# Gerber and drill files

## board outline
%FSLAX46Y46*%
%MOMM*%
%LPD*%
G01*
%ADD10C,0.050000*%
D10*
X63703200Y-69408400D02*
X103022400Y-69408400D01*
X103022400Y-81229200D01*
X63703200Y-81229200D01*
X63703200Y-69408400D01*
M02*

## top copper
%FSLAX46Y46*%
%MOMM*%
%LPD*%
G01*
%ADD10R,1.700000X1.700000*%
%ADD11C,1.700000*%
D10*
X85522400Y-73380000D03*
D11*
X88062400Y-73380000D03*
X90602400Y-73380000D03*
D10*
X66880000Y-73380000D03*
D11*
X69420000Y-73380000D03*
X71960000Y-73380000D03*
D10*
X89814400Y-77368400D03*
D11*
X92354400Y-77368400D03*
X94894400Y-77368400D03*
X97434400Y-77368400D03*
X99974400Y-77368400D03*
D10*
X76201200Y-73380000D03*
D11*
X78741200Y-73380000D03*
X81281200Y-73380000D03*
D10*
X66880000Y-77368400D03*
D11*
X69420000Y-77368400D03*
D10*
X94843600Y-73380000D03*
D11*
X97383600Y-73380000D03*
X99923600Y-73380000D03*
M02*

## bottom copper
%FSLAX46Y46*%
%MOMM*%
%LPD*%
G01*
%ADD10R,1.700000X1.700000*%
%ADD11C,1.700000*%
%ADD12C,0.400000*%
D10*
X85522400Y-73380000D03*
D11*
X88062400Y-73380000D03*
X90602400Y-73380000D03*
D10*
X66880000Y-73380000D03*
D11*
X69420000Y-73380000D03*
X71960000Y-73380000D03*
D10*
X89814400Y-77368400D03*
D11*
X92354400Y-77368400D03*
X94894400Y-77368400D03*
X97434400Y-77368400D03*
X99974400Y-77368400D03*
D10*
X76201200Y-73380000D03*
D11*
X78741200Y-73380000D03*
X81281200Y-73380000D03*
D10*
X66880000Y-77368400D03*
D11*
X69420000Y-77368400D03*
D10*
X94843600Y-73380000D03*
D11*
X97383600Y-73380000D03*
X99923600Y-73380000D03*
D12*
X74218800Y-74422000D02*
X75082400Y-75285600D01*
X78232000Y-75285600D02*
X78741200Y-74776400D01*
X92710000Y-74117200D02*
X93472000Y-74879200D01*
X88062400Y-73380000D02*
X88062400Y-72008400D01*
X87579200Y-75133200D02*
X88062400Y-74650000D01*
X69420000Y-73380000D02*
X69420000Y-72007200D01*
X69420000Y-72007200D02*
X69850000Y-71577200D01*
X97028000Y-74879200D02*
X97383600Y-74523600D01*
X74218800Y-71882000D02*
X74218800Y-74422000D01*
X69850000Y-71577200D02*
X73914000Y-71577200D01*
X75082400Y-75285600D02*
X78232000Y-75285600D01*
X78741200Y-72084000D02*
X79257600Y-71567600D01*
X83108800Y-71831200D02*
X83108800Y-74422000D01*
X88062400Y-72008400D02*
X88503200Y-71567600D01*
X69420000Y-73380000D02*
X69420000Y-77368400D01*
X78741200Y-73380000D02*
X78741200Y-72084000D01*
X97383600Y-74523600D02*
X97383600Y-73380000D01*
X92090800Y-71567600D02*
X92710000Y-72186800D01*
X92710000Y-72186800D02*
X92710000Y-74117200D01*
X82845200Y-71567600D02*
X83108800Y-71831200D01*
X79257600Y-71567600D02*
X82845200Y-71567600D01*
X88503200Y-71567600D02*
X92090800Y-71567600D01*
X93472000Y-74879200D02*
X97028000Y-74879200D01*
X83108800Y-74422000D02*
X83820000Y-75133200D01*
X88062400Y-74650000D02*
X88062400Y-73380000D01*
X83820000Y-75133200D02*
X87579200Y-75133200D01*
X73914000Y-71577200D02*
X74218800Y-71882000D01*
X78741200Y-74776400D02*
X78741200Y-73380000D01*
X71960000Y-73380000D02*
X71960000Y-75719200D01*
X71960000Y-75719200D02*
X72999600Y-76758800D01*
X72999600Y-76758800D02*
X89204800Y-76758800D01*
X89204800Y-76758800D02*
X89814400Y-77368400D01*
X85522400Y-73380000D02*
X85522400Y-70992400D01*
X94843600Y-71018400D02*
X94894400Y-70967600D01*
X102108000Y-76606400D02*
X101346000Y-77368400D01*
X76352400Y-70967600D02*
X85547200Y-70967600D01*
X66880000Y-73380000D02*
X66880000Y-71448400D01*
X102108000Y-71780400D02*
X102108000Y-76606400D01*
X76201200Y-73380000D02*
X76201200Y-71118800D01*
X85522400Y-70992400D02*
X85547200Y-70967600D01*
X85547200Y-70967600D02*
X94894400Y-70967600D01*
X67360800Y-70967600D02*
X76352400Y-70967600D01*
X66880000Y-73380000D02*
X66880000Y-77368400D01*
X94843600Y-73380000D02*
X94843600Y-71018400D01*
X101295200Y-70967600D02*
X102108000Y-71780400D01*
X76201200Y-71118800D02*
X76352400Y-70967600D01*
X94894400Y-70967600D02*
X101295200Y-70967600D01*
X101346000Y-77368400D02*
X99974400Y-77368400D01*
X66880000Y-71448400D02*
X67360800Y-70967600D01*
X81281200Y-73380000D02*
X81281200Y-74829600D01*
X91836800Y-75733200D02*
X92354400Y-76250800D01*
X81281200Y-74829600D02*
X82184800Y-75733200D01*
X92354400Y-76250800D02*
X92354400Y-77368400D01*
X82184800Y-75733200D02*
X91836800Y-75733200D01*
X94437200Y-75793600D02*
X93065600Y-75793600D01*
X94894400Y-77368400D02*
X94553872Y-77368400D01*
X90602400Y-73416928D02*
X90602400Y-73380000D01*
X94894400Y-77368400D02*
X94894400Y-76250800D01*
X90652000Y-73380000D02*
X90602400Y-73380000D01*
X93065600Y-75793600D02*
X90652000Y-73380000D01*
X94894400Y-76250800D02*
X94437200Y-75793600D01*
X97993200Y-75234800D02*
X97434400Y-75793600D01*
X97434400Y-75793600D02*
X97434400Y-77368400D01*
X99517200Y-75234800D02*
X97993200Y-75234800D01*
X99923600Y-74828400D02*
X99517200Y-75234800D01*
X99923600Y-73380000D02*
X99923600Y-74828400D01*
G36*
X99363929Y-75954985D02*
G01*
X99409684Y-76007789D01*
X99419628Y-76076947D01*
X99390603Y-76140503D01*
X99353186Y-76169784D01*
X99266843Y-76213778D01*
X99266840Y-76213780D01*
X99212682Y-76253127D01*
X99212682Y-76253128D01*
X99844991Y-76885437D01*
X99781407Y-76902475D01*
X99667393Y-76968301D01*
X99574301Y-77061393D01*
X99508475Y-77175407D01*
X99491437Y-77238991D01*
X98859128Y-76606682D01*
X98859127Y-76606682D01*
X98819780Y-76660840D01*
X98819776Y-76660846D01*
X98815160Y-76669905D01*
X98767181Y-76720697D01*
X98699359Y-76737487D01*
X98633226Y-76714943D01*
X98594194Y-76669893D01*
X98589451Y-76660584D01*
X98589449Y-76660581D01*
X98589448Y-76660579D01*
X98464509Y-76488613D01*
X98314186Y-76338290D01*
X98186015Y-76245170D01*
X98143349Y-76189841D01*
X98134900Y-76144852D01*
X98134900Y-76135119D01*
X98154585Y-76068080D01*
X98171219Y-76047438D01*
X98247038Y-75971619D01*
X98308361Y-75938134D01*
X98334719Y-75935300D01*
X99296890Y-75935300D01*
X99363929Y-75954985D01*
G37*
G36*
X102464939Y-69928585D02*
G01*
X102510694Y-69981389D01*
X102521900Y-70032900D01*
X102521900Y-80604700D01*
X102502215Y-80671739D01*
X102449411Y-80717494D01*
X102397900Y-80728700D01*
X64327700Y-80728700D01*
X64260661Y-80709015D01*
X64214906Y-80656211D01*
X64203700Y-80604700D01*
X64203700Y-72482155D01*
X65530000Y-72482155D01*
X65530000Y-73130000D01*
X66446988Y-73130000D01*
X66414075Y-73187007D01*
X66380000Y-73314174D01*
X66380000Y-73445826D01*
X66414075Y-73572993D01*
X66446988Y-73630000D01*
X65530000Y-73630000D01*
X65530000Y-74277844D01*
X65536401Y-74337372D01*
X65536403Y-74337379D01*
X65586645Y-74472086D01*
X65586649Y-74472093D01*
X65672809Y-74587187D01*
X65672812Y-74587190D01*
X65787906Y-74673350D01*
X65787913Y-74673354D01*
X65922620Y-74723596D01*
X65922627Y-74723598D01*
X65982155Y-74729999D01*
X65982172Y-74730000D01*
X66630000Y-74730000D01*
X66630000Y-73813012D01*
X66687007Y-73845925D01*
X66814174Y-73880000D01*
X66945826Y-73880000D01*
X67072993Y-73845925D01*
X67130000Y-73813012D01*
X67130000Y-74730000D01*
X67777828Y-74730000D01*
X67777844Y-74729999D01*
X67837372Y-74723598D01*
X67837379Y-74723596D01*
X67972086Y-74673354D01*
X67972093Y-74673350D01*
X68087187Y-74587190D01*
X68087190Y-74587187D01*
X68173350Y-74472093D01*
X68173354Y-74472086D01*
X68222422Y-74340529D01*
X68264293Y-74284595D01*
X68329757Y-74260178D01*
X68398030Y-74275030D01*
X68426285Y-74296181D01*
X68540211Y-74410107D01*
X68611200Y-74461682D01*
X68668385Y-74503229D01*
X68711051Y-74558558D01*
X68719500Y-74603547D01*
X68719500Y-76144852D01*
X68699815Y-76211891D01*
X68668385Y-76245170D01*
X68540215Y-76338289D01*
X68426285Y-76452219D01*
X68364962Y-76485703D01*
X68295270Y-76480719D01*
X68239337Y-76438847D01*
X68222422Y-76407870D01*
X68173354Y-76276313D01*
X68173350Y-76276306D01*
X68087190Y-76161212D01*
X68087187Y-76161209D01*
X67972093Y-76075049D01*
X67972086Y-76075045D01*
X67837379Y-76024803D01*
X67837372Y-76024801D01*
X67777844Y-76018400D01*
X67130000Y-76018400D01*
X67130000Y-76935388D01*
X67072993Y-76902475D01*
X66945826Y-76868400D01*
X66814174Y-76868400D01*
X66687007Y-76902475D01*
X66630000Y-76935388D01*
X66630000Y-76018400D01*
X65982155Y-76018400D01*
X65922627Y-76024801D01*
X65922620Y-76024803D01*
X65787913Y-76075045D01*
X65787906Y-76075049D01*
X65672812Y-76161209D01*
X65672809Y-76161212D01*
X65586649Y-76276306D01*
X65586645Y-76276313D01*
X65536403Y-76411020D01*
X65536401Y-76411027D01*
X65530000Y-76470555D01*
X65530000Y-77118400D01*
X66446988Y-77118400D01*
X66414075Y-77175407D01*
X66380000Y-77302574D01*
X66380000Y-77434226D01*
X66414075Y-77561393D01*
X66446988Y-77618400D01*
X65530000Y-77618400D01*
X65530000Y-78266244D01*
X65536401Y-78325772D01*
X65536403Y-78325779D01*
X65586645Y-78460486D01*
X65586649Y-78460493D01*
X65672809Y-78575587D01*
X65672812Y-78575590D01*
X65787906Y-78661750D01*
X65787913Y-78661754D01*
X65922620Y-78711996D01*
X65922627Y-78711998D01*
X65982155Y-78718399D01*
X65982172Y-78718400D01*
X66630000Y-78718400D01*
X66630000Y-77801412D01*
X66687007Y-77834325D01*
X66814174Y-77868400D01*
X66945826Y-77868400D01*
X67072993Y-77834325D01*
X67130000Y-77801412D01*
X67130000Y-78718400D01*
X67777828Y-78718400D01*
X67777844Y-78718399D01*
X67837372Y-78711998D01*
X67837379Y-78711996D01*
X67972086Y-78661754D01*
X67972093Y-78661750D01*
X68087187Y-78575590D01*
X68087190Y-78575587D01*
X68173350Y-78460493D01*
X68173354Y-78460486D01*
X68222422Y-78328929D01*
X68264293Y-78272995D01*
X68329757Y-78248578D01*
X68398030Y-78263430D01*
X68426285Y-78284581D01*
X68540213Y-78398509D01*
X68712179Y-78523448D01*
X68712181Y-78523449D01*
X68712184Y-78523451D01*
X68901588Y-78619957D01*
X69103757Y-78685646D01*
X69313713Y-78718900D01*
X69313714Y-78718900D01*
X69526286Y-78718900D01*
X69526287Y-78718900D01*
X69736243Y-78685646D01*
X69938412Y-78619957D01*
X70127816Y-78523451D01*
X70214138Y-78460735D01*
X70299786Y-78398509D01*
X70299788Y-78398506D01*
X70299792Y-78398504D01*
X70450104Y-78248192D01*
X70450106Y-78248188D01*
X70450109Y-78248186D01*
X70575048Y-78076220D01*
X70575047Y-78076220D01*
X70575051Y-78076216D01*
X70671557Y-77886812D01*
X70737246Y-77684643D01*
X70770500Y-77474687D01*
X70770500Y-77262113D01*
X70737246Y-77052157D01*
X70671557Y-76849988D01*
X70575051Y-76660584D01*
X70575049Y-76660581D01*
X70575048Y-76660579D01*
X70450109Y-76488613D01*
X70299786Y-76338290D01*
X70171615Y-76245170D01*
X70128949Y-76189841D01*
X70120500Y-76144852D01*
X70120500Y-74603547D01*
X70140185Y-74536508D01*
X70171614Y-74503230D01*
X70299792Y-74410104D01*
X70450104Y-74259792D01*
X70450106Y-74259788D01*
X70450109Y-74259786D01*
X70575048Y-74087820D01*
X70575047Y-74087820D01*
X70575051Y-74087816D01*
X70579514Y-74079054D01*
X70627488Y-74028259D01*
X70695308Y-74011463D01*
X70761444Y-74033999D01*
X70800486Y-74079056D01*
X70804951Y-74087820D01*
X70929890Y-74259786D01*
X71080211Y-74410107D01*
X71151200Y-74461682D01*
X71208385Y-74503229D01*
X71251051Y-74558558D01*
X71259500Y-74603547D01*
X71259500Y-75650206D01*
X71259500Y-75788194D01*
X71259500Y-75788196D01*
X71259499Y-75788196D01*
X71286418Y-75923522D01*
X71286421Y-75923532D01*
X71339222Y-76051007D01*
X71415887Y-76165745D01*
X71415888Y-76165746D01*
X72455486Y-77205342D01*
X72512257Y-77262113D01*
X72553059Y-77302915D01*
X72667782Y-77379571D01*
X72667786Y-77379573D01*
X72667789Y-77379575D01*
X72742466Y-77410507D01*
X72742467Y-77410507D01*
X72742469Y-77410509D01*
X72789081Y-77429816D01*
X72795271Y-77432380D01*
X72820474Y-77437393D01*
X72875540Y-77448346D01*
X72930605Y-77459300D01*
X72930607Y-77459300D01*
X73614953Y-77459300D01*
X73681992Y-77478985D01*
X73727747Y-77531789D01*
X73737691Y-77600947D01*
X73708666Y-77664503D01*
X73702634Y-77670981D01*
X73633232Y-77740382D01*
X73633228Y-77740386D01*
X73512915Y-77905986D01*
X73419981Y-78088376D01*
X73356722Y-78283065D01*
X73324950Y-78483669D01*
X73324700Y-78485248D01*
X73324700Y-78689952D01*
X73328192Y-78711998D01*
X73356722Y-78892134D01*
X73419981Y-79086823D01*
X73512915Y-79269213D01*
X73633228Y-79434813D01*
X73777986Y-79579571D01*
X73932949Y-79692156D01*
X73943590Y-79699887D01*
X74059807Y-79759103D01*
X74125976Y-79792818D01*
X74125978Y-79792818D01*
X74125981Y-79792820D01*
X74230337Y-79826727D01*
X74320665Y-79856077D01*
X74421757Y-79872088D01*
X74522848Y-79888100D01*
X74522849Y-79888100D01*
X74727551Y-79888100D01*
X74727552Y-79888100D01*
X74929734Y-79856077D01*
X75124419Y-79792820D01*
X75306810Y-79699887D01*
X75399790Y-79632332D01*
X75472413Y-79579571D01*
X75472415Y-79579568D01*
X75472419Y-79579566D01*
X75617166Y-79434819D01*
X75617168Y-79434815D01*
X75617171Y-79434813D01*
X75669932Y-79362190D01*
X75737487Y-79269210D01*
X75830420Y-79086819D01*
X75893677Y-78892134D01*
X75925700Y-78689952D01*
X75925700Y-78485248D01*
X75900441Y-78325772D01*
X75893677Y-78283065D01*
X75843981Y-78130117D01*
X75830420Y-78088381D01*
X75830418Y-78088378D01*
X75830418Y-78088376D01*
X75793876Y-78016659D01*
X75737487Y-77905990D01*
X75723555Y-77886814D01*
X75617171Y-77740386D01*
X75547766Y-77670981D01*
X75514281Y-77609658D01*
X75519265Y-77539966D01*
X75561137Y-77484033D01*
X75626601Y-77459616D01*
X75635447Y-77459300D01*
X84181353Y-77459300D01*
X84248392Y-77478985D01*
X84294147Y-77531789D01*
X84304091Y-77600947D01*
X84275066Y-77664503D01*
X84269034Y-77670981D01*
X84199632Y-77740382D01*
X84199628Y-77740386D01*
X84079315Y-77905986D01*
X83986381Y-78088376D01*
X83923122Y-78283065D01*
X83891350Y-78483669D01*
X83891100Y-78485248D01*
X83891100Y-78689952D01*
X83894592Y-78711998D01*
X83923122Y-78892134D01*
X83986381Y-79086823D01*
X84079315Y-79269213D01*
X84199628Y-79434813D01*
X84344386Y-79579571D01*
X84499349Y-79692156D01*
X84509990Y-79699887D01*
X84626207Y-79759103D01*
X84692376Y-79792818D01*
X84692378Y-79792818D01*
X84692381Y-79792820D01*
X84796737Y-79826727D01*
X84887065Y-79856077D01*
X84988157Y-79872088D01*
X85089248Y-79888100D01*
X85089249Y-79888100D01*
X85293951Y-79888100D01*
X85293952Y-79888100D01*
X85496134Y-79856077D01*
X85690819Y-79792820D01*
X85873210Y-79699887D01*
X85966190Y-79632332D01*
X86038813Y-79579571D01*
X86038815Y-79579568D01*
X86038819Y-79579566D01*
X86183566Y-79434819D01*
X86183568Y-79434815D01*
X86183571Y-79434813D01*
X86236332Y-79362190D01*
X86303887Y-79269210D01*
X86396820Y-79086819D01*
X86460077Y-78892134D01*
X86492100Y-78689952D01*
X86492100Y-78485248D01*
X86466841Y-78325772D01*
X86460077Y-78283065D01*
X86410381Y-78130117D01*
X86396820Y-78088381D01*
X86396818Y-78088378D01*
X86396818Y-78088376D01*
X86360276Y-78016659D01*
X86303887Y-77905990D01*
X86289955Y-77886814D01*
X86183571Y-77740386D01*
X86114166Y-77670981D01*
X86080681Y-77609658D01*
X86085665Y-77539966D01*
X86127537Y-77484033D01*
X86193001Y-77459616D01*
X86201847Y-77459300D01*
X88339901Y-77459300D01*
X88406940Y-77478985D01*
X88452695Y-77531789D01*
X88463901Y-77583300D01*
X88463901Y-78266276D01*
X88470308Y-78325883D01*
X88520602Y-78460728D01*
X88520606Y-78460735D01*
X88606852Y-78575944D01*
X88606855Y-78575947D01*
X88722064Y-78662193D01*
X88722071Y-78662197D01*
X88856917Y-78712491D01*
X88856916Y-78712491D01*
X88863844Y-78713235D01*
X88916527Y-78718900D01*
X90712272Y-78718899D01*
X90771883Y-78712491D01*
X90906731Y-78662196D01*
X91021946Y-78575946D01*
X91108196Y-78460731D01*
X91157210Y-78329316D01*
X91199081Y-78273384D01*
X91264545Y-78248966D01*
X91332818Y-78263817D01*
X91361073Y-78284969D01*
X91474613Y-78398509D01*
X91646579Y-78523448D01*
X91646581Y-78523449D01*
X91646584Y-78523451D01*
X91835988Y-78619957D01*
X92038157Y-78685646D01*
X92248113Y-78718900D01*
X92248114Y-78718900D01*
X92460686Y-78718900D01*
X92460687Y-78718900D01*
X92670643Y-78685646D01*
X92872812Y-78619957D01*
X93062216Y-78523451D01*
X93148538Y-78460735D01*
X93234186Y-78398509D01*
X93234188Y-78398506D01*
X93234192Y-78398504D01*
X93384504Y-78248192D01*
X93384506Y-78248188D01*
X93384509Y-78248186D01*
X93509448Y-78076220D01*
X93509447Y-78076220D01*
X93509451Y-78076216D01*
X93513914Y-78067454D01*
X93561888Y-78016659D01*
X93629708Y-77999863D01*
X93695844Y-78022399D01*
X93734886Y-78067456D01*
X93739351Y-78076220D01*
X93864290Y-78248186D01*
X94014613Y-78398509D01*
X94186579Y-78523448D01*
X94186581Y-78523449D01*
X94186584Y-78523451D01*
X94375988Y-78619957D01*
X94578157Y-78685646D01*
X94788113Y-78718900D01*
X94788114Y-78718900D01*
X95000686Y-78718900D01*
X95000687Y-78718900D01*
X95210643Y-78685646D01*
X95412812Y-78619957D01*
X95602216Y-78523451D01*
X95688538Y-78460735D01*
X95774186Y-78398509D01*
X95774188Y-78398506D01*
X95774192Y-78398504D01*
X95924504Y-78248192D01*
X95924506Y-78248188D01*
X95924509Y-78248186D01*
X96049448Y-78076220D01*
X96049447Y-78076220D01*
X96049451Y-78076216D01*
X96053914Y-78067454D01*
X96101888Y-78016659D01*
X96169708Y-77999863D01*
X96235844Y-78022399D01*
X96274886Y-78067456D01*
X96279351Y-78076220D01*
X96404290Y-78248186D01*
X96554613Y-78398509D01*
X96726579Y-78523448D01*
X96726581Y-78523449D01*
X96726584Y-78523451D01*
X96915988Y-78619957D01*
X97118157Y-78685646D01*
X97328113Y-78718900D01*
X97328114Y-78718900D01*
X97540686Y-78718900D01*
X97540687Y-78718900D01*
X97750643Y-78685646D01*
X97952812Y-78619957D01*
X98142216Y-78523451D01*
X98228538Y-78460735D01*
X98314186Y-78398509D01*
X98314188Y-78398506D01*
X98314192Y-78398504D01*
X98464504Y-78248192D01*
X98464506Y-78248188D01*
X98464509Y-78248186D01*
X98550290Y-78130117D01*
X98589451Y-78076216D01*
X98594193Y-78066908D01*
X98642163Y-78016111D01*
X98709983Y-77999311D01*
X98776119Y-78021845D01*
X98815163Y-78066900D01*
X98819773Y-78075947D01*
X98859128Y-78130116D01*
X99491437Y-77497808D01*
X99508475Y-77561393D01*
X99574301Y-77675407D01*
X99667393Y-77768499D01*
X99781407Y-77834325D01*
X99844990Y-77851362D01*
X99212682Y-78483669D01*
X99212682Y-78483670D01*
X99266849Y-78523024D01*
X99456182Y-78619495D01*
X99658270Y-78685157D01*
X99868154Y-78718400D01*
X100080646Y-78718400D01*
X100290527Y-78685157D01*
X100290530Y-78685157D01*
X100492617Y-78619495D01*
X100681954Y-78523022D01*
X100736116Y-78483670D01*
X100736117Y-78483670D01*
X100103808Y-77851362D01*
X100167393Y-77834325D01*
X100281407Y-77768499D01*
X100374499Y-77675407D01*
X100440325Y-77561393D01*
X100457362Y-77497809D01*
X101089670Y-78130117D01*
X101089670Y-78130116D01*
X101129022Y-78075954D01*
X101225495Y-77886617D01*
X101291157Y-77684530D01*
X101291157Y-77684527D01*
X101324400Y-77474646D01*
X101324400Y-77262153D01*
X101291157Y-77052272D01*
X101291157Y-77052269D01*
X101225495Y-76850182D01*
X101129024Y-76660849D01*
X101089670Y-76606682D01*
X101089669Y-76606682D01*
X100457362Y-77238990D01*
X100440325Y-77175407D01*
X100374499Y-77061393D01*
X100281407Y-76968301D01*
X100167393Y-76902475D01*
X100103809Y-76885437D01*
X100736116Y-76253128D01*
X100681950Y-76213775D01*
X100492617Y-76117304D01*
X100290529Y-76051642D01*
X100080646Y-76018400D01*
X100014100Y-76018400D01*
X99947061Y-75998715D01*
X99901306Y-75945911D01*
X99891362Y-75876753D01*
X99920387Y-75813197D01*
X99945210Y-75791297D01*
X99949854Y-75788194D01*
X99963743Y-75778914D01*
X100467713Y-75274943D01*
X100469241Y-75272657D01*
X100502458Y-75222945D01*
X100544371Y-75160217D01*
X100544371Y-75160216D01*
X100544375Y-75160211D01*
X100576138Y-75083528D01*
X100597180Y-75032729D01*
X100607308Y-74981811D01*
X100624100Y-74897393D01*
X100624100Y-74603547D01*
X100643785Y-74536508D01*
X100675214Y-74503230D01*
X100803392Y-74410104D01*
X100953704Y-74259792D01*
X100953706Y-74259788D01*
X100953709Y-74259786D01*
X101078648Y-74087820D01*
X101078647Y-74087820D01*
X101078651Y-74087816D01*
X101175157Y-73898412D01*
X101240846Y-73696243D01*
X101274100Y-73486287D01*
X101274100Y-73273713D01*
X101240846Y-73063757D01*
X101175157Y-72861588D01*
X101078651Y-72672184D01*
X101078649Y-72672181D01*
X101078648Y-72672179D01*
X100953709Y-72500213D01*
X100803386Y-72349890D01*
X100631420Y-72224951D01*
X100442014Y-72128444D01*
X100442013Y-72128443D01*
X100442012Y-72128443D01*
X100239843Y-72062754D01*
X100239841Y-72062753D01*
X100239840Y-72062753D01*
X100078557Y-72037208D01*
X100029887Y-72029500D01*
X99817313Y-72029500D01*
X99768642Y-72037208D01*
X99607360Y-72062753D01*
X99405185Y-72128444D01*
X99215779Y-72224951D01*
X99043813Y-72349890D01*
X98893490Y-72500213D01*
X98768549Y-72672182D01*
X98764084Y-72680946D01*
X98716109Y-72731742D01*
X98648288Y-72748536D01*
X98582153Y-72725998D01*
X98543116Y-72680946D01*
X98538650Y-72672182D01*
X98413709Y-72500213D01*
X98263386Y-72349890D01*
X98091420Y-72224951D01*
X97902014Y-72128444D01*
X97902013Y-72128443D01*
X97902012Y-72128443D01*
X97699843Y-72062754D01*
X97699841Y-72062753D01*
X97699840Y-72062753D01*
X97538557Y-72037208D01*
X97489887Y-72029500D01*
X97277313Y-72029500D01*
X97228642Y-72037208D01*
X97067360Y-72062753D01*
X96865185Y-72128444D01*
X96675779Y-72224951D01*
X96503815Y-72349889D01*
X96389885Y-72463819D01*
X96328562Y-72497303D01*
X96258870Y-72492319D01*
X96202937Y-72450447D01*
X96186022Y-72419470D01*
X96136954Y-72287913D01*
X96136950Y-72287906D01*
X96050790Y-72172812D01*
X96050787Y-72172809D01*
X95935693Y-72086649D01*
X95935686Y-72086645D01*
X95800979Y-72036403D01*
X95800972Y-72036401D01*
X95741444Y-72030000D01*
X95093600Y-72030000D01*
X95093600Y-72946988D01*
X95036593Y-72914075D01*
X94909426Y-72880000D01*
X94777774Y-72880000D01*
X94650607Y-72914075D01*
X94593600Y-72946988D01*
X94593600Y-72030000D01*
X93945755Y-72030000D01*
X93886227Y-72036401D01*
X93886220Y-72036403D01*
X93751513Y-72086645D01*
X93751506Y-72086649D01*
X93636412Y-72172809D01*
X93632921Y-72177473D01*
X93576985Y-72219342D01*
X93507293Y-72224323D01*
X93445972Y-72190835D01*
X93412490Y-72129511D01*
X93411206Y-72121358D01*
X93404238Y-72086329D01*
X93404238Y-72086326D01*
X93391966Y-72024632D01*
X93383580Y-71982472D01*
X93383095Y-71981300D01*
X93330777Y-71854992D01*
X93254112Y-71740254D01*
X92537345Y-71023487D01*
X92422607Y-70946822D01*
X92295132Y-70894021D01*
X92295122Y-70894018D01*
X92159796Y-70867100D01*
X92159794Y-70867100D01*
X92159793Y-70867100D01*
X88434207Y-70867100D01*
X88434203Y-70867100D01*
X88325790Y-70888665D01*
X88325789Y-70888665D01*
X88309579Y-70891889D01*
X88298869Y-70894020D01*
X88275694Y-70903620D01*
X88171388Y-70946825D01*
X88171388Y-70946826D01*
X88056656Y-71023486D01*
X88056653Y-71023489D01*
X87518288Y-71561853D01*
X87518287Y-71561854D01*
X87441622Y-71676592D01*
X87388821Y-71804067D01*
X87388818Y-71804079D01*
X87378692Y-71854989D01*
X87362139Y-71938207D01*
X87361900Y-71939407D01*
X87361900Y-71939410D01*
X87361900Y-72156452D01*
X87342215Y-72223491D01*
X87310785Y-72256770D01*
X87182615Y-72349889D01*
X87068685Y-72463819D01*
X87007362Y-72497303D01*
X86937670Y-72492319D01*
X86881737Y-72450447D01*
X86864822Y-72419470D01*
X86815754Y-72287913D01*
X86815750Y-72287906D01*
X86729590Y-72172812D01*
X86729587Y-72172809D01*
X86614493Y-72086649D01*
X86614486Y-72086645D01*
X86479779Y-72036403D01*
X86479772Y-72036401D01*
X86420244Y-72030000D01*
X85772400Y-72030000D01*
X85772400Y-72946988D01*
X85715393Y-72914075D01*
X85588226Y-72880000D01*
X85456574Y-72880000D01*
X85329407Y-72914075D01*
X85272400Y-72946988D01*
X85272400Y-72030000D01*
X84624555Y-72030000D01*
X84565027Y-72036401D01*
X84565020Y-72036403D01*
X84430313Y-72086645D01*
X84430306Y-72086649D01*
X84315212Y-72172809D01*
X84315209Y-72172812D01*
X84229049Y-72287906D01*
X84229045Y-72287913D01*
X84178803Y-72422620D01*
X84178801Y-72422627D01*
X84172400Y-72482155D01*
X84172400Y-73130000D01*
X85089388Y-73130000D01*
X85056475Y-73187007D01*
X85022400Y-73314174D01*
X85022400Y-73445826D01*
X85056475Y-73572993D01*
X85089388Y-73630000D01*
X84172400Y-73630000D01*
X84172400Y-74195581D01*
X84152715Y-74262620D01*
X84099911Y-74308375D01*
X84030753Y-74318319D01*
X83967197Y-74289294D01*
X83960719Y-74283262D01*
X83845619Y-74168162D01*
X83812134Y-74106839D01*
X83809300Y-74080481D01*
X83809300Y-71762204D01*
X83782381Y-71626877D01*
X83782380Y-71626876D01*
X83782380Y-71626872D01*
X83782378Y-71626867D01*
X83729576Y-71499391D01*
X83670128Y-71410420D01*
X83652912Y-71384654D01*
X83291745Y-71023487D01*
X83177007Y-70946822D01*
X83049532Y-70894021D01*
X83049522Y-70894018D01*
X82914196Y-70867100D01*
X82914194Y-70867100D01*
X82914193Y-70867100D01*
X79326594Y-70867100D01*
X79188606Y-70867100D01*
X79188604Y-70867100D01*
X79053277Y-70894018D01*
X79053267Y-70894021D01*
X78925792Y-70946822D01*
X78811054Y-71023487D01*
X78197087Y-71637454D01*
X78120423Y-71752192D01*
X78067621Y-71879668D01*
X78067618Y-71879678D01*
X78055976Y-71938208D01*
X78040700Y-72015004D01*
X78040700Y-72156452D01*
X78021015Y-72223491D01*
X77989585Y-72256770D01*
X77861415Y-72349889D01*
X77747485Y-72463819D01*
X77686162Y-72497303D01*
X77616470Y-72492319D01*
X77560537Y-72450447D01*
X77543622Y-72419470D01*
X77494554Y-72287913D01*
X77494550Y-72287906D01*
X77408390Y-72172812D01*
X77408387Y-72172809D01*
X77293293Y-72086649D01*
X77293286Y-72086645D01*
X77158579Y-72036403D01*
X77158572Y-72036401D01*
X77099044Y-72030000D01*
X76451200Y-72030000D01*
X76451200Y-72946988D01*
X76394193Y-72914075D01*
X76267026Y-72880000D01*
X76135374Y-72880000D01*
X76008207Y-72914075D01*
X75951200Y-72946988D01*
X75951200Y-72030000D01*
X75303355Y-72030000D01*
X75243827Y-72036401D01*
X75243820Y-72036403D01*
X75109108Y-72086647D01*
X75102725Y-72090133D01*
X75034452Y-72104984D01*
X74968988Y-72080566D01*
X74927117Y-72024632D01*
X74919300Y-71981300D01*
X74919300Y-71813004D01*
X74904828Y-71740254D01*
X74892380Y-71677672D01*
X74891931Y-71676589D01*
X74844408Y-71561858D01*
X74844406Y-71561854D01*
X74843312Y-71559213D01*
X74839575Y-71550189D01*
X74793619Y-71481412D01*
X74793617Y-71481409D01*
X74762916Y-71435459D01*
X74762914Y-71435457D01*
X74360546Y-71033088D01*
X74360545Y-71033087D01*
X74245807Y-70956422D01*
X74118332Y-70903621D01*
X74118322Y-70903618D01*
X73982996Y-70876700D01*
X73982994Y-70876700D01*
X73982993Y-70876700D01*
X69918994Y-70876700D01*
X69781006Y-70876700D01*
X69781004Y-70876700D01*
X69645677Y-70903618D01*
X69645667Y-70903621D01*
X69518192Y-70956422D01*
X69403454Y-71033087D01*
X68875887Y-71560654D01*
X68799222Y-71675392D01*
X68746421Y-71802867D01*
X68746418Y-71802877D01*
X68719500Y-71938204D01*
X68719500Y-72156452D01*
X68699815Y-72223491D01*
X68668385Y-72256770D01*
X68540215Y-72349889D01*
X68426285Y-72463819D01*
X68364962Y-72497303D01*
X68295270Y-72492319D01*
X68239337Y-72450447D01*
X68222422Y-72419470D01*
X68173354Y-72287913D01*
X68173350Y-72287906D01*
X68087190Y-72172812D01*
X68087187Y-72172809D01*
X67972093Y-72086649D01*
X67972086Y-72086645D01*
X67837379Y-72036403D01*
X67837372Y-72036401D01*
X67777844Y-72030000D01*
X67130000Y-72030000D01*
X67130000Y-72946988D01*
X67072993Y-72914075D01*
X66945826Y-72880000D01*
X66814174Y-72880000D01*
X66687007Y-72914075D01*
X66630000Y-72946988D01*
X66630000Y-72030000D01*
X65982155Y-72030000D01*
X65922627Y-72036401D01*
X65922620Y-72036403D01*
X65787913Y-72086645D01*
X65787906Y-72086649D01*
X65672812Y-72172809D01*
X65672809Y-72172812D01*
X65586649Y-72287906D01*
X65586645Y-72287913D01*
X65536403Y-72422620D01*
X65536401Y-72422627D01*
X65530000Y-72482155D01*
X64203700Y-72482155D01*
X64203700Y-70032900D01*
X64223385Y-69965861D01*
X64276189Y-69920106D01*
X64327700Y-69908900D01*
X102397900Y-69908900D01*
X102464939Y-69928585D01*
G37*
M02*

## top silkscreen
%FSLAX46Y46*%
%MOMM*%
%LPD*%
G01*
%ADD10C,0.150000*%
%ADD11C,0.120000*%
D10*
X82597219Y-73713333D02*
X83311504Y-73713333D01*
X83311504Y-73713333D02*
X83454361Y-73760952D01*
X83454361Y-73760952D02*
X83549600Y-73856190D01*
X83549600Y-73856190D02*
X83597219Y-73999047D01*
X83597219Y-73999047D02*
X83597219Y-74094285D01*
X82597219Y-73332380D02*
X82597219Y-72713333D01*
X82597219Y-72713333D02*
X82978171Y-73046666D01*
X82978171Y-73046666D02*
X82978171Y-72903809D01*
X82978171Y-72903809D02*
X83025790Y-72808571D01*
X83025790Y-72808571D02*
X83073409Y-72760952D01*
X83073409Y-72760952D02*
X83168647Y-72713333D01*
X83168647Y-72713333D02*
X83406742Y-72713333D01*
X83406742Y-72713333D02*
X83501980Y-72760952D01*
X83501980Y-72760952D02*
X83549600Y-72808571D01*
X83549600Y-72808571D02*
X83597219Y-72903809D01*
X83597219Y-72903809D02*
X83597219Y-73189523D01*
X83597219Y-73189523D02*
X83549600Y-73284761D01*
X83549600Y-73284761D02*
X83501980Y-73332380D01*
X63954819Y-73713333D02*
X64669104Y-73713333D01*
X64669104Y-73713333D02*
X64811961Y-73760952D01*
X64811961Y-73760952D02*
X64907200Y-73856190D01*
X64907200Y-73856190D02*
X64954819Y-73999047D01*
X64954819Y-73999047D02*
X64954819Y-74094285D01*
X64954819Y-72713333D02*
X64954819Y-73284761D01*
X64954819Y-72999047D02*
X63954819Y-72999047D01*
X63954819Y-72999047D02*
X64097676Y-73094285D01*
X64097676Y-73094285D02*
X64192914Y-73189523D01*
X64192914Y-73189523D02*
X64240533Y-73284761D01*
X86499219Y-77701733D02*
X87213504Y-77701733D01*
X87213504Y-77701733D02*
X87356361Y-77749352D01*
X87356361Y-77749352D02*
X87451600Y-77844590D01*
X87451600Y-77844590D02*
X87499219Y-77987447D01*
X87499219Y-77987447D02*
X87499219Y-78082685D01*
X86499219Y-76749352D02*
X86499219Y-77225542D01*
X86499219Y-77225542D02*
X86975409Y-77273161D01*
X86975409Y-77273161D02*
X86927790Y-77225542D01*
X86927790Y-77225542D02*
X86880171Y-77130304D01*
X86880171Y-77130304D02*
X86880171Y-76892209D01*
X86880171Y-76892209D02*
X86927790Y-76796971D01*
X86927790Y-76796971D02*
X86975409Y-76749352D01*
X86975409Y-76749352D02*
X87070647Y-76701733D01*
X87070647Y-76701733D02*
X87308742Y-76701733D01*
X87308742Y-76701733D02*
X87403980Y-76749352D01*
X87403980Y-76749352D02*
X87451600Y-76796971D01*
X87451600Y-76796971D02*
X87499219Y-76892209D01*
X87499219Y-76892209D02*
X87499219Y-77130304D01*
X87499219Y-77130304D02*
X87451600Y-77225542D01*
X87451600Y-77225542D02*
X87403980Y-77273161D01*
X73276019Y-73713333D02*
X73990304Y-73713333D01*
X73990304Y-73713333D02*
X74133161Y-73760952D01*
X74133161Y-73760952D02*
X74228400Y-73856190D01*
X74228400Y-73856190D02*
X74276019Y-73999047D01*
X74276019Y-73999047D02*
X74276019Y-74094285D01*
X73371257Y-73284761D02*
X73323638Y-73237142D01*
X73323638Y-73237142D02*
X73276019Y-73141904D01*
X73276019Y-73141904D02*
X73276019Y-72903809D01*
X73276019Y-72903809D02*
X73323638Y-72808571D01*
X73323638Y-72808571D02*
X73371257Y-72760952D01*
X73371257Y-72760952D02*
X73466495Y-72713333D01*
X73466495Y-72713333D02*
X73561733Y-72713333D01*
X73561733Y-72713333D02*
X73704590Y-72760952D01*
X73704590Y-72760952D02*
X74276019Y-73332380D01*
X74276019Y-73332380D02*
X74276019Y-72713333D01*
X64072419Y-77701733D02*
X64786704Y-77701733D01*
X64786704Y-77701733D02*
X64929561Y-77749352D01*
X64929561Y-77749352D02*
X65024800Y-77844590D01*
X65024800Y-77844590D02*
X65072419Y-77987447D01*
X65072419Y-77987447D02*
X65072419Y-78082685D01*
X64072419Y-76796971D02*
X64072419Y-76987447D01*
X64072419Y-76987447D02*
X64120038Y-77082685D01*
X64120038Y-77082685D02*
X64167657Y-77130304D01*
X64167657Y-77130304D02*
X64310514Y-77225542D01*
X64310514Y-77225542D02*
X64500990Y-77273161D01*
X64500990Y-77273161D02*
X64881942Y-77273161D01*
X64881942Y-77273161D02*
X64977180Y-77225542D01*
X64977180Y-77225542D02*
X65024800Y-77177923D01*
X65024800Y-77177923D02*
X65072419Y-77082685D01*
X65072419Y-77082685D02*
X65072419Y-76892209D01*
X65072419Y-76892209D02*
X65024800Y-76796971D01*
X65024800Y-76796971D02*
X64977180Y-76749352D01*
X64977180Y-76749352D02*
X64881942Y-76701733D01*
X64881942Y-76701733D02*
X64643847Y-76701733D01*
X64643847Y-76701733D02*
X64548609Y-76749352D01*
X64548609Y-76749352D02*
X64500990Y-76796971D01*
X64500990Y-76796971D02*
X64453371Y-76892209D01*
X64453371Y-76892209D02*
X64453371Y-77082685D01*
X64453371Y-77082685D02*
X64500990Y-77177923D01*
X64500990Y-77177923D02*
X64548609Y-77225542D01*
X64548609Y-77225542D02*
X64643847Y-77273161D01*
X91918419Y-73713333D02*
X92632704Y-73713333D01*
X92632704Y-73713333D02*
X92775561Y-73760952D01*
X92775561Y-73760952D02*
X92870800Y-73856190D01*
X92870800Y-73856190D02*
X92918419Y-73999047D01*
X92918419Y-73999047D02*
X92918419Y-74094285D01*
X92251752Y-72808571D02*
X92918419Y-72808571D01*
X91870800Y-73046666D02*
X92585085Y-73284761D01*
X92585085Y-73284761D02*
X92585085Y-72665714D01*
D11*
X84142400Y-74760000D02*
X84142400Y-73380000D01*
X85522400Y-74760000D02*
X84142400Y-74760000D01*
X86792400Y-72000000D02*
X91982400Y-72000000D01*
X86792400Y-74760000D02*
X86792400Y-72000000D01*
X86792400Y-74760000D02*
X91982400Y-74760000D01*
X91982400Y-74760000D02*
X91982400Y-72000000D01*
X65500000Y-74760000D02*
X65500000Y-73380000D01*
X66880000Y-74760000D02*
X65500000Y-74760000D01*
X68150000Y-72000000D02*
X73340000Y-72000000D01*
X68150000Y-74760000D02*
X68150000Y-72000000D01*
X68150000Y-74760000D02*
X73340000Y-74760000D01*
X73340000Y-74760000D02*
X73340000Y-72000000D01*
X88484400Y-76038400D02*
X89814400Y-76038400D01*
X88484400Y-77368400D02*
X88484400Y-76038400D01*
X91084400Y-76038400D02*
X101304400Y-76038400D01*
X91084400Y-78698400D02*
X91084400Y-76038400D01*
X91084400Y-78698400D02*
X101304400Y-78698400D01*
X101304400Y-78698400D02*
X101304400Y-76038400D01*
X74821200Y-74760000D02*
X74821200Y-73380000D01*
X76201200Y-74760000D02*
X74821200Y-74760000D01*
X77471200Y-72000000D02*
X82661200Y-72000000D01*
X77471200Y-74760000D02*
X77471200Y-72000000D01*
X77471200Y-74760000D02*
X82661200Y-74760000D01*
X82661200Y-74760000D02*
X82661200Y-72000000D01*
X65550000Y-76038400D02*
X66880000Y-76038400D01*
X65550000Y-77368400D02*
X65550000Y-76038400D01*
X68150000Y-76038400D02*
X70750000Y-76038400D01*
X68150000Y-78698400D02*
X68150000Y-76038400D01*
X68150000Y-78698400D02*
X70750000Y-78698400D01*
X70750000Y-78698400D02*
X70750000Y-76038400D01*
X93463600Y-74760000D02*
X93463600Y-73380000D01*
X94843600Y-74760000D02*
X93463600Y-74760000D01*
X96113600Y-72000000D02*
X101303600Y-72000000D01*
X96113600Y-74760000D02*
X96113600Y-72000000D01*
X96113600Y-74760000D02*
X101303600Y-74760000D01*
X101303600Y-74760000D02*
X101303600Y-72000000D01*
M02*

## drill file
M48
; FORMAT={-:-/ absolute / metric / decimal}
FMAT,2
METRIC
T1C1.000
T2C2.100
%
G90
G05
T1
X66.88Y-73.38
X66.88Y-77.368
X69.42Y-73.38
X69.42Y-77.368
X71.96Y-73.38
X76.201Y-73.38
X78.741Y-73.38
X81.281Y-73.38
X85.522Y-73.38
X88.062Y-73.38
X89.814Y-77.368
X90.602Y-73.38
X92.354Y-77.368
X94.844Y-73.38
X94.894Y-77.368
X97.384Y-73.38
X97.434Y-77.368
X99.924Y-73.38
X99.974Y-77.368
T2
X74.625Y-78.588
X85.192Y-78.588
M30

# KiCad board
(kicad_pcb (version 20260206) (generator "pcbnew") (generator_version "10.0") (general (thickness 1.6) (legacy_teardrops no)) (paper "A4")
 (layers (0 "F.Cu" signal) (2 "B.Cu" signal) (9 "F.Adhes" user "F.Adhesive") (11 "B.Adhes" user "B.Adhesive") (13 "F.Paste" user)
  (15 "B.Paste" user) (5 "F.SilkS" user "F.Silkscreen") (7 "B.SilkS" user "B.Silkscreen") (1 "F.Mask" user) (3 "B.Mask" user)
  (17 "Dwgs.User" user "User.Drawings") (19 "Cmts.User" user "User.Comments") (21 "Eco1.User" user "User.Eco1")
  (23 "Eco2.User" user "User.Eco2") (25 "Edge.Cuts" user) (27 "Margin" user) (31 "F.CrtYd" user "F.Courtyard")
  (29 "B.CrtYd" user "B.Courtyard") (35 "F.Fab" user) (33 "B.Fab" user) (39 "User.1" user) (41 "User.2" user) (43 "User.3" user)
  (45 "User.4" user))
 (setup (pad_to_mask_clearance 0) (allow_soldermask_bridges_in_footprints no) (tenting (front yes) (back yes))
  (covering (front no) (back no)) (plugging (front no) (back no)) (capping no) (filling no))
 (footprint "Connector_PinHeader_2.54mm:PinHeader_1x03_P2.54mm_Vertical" (layer "F.Cu") (at 85.5224 73.38 90)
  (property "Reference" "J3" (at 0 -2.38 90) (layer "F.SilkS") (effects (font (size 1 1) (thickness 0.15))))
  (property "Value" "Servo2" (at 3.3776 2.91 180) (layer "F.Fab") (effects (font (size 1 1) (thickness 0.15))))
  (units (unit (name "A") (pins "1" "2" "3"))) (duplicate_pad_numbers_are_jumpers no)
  (fp_line (start -1.38 -1.38) (end 0 -1.38) (stroke (width 0.12) (type solid)) (layer "F.SilkS"))
  (fp_line (start -1.38 0) (end -1.38 -1.38) (stroke (width 0.12) (type solid)) (layer "F.SilkS"))
  (fp_line (start 1.38 1.27) (end 1.38 6.46) (stroke (width 0.12) (type solid)) (layer "F.SilkS"))
  (fp_line (start -1.38 1.27) (end 1.38 1.27) (stroke (width 0.12) (type solid)) (layer "F.SilkS"))
  (fp_line (start -1.38 1.27) (end -1.38 6.46) (stroke (width 0.12) (type solid)) (layer "F.SilkS"))
  (fp_line (start -1.38 6.46) (end 1.38 6.46) (stroke (width 0.12) (type solid)) (layer "F.SilkS"))
  (pad "1" thru_hole rect (at 0 0 90) (size 1.7 1.7) (drill 1) (layers "*.Cu" "*.Mask") (remove_unused_layers no) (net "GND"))
  (pad "2" thru_hole circle (at 0 2.54 90) (size 1.7 1.7) (drill 1) (layers "*.Cu" "*.Mask") (remove_unused_layers no) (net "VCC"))
  (pad "3" thru_hole circle (at 0 5.08 90) (size 1.7 1.7) (drill 1) (layers "*.Cu" "*.Mask") (remove_unused_layers no) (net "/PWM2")))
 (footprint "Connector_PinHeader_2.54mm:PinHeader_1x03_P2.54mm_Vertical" (layer "F.Cu") (at 66.88 73.38 90)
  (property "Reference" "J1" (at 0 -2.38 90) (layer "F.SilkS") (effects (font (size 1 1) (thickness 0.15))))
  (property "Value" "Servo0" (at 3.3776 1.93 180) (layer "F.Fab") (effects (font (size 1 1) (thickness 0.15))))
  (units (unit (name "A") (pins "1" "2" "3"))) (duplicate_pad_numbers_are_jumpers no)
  (fp_line (start -1.38 -1.38) (end 0 -1.38) (stroke (width 0.12) (type solid)) (layer "F.SilkS"))
  (fp_line (start -1.38 0) (end -1.38 -1.38) (stroke (width 0.12) (type solid)) (layer "F.SilkS"))
  (fp_line (start 1.38 1.27) (end 1.38 6.46) (stroke (width 0.12) (type solid)) (layer "F.SilkS"))
  (fp_line (start -1.38 1.27) (end 1.38 1.27) (stroke (width 0.12) (type solid)) (layer "F.SilkS"))
  (fp_line (start -1.38 1.27) (end -1.38 6.46) (stroke (width 0.12) (type solid)) (layer "F.SilkS"))
  (fp_line (start -1.38 6.46) (end 1.38 6.46) (stroke (width 0.12) (type solid)) (layer "F.SilkS"))
  (pad "1" thru_hole rect (at 0 0 90) (size 1.7 1.7) (drill 1) (layers "*.Cu" "*.Mask") (remove_unused_layers no) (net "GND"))
  (pad "2" thru_hole circle (at 0 2.54 90) (size 1.7 1.7) (drill 1) (layers "*.Cu" "*.Mask") (remove_unused_layers no) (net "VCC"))
  (pad "3" thru_hole circle (at 0 5.08 90) (size 1.7 1.7) (drill 1) (layers "*.Cu" "*.Mask") (remove_unused_layers no) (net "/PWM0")))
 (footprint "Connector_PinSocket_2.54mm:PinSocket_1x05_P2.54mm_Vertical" (layer "F.Cu") (at 89.8144 77.3684 90)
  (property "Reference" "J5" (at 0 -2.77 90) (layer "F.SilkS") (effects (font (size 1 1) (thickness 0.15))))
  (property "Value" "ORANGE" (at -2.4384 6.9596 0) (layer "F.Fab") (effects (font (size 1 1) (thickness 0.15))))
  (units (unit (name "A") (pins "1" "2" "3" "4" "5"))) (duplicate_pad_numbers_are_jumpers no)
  (fp_line (start 1.33 -1.33) (end 1.33 0) (stroke (width 0.12) (type solid)) (layer "F.SilkS"))
  (fp_line (start 0 -1.33) (end 1.33 -1.33) (stroke (width 0.12) (type solid)) (layer "F.SilkS"))
  (fp_line (start 1.33 1.27) (end 1.33 11.49) (stroke (width 0.12) (type solid)) (layer "F.SilkS"))
  (fp_line (start -1.33 1.27) (end 1.33 1.27) (stroke (width 0.12) (type solid)) (layer "F.SilkS"))
  (fp_line (start -1.33 1.27) (end -1.33 11.49) (stroke (width 0.12) (type solid)) (layer "F.SilkS"))
  (fp_line (start -1.33 11.49) (end 1.33 11.49) (stroke (width 0.12) (type solid)) (layer "F.SilkS"))
  (pad "1" thru_hole rect (at 0 0 90) (size 1.7 1.7) (drill 1) (layers "*.Cu" "*.Mask") (remove_unused_layers no) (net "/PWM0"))
  (pad "2" thru_hole circle (at 0 2.54 90) (size 1.7 1.7) (drill 1) (layers "*.Cu" "*.Mask") (remove_unused_layers no) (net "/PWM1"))
  (pad "3" thru_hole circle (at 0 5.08 90) (size 1.7 1.7) (drill 1) (layers "*.Cu" "*.Mask") (remove_unused_layers no) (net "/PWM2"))
  (pad "4" thru_hole circle (at 0 7.62 90) (size 1.7 1.7) (drill 1) (layers "*.Cu" "*.Mask") (remove_unused_layers no) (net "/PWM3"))
  (pad "5" thru_hole circle (at 0 10.16 90) (size 1.7 1.7) (drill 1) (layers "*.Cu" "*.Mask") (remove_unused_layers no) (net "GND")))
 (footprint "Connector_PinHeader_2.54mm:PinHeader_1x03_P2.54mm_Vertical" (layer "F.Cu") (at 76.2012 73.38 90)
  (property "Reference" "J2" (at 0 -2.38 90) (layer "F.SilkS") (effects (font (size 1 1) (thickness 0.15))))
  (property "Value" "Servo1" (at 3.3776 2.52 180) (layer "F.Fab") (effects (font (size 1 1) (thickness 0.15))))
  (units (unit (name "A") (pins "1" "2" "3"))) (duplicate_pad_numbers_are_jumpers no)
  (fp_line (start -1.38 -1.38) (end 0 -1.38) (stroke (width 0.12) (type solid)) (layer "F.SilkS"))
  (fp_line (start -1.38 0) (end -1.38 -1.38) (stroke (width 0.12) (type solid)) (layer "F.SilkS"))
  (fp_line (start 1.38 1.27) (end 1.38 6.46) (stroke (width 0.12) (type solid)) (layer "F.SilkS"))
  (fp_line (start -1.38 1.27) (end 1.38 1.27) (stroke (width 0.12) (type solid)) (layer "F.SilkS"))
  (fp_line (start -1.38 1.27) (end -1.38 6.46) (stroke (width 0.12) (type solid)) (layer "F.SilkS"))
  (fp_line (start -1.38 6.46) (end 1.38 6.46) (stroke (width 0.12) (type solid)) (layer "F.SilkS"))
  (pad "1" thru_hole rect (at 0 0 90) (size 1.7 1.7) (drill 1) (layers "*.Cu" "*.Mask") (remove_unused_layers no) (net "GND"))
  (pad "2" thru_hole circle (at 0 2.54 90) (size 1.7 1.7) (drill 1) (layers "*.Cu" "*.Mask") (remove_unused_layers no) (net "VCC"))
  (pad "3" thru_hole circle (at 0 5.08 90) (size 1.7 1.7) (drill 1) (layers "*.Cu" "*.Mask") (remove_unused_layers no) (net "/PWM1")))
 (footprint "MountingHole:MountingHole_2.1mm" (layer "F.Cu") (at 74.6252 78.5876)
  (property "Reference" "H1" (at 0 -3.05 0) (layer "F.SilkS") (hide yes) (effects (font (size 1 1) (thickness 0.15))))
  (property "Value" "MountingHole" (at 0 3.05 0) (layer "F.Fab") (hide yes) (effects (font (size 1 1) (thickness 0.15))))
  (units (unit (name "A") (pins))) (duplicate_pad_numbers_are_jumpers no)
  (pad "" np_thru_hole circle (at 0 0) (size 2.1 2.1) (drill 2.1) (layers "*.Cu" "*.Mask")))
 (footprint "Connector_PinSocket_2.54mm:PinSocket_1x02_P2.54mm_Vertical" (layer "F.Cu") (at 66.88 77.3684 90)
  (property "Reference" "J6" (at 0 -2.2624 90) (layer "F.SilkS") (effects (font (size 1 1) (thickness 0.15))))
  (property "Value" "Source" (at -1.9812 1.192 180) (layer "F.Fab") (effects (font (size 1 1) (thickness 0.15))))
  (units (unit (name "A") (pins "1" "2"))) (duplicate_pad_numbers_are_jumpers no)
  (fp_line (start 1.33 -1.33) (end 1.33 0) (stroke (width 0.12) (type solid)) (layer "F.SilkS"))
  (fp_line (start 0 -1.33) (end 1.33 -1.33) (stroke (width 0.12) (type solid)) (layer "F.SilkS"))
  (fp_line (start 1.33 1.27) (end 1.33 3.87) (stroke (width 0.12) (type solid)) (layer "F.SilkS"))
  (fp_line (start -1.33 1.27) (end 1.33 1.27) (stroke (width 0.12) (type solid)) (layer "F.SilkS"))
  (fp_line (start -1.33 1.27) (end -1.33 3.87) (stroke (width 0.12) (type solid)) (layer "F.SilkS"))
  (fp_line (start -1.33 3.87) (end 1.33 3.87) (stroke (width 0.12) (type solid)) (layer "F.SilkS"))
  (pad "1" thru_hole rect (at 0 0 90) (size 1.7 1.7) (drill 1) (layers "*.Cu" "*.Mask") (remove_unused_layers no) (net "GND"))
  (pad "2" thru_hole circle (at 0 2.54 90) (size 1.7 1.7) (drill 1) (layers "*.Cu" "*.Mask") (remove_unused_layers no) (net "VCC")))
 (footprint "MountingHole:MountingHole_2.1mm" (layer "F.Cu") (at 85.1916 78.5876)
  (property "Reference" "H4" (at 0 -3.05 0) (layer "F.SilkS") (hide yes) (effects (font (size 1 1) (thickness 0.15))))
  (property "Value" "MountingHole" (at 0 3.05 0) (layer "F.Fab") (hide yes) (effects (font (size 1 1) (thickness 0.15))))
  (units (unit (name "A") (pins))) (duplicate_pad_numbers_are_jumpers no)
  (pad "" np_thru_hole circle (at 0 0) (size 2.1 2.1) (drill 2.1) (layers "*.Cu" "*.Mask")))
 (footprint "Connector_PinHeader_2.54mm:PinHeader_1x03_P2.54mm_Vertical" (layer "F.Cu") (at 94.8436 73.38 90)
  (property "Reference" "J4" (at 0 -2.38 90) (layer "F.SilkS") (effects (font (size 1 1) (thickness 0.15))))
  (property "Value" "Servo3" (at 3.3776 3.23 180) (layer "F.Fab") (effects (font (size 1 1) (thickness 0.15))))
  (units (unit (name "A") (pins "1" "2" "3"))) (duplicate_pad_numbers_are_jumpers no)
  (fp_line (start -1.38 -1.38) (end 0 -1.38) (stroke (width 0.12) (type solid)) (layer "F.SilkS"))
  (fp_line (start -1.38 0) (end -1.38 -1.38) (stroke (width 0.12) (type solid)) (layer "F.SilkS"))
  (fp_line (start 1.38 1.27) (end 1.38 6.46) (stroke (width 0.12) (type solid)) (layer "F.SilkS"))
  (fp_line (start -1.38 1.27) (end 1.38 1.27) (stroke (width 0.12) (type solid)) (layer "F.SilkS"))
  (fp_line (start -1.38 1.27) (end -1.38 6.46) (stroke (width 0.12) (type solid)) (layer "F.SilkS"))
  (fp_line (start -1.38 6.46) (end 1.38 6.46) (stroke (width 0.12) (type solid)) (layer "F.SilkS"))
  (pad "1" thru_hole rect (at 0 0 90) (size 1.7 1.7) (drill 1) (layers "*.Cu" "*.Mask") (remove_unused_layers no) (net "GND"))
  (pad "2" thru_hole circle (at 0 2.54 90) (size 1.7 1.7) (drill 1) (layers "*.Cu" "*.Mask") (remove_unused_layers no) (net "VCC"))
  (pad "3" thru_hole circle (at 0 5.08 90) (size 1.7 1.7) (drill 1) (layers "*.Cu" "*.Mask") (remove_unused_layers no) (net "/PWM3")))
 (gr_rect (start 63.7032 69.4084) (end 103.0224 81.2292) (stroke (width 0.05) (type default)) (fill no) (layer "Edge.Cuts"))
 (segment (start 74.2188 74.422) (end 75.0824 75.2856) (width 0.4) (layer "B.Cu") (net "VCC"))
 (segment (start 78.232 75.2856) (end 78.7412 74.7764) (width 0.4) (layer "B.Cu") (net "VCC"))
 (segment (start 92.71 74.1172) (end 93.472 74.8792) (width 0.4) (layer "B.Cu") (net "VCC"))
 (segment (start 88.0624 73.38) (end 88.0624 72.0084) (width 0.4) (layer "B.Cu") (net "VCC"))
 (segment (start 87.5792 75.1332) (end 88.0624 74.65) (width 0.4) (layer "B.Cu") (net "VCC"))
 (segment (start 69.42 73.38) (end 69.42 72.0072) (width 0.4) (layer "B.Cu") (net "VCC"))
 (segment (start 69.42 72.0072) (end 69.85 71.5772) (width 0.4) (layer "B.Cu") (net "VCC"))
 (segment (start 97.028 74.8792) (end 97.3836 74.5236) (width 0.4) (layer "B.Cu") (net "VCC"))
 (segment (start 74.2188 71.882) (end 74.2188 74.422) (width 0.4) (layer "B.Cu") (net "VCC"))
 (segment (start 69.85 71.5772) (end 73.914 71.5772) (width 0.4) (layer "B.Cu") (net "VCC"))
 (segment (start 75.0824 75.2856) (end 78.232 75.2856) (width 0.4) (layer "B.Cu") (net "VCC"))
 (segment (start 78.7412 72.084) (end 79.2576 71.5676) (width 0.4) (layer "B.Cu") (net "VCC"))
 (segment (start 83.1088 71.8312) (end 83.1088 74.422) (width 0.4) (layer "B.Cu") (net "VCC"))
 (segment (start 88.0624 72.0084) (end 88.5032 71.5676) (width 0.4) (layer "B.Cu") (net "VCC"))
 (segment (start 69.42 73.38) (end 69.42 77.3684) (width 0.4) (layer "B.Cu") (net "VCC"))
 (segment (start 78.7412 73.38) (end 78.7412 72.084) (width 0.4) (layer "B.Cu") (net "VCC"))
 (segment (start 97.3836 74.5236) (end 97.3836 73.38) (width 0.4) (layer "B.Cu") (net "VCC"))
 (segment (start 92.0908 71.5676) (end 92.71 72.1868) (width 0.4) (layer "B.Cu") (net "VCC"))
 (segment (start 92.71 72.1868) (end 92.71 74.1172) (width 0.4) (layer "B.Cu") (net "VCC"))
 (segment (start 82.8452 71.5676) (end 83.1088 71.8312) (width 0.4) (layer "B.Cu") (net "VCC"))
 (segment (start 79.2576 71.5676) (end 82.8452 71.5676) (width 0.4) (layer "B.Cu") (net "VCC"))
 (segment (start 88.5032 71.5676) (end 92.0908 71.5676) (width 0.4) (layer "B.Cu") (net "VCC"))
 (segment (start 93.472 74.8792) (end 97.028 74.8792) (width 0.4) (layer "B.Cu") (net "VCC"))
 (segment (start 83.1088 74.422) (end 83.82 75.1332) (width 0.4) (layer "B.Cu") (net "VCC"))
 (segment (start 88.0624 74.65) (end 88.0624 73.38) (width 0.4) (layer "B.Cu") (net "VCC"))
 (segment (start 83.82 75.1332) (end 87.5792 75.1332) (width 0.4) (layer "B.Cu") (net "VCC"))
 (segment (start 73.914 71.5772) (end 74.2188 71.882) (width 0.4) (layer "B.Cu") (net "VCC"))
 (segment (start 78.7412 74.7764) (end 78.7412 73.38) (width 0.4) (layer "B.Cu") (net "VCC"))
 (segment (start 71.96 73.38) (end 71.96 75.7192) (width 0.4) (layer "B.Cu") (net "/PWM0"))
 (segment (start 71.96 75.7192) (end 72.9996 76.7588) (width 0.4) (layer "B.Cu") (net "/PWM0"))
 (segment (start 72.9996 76.7588) (end 89.2048 76.7588) (width 0.4) (layer "B.Cu") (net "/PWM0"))
 (segment (start 89.2048 76.7588) (end 89.8144 77.3684) (width 0.4) (layer "B.Cu") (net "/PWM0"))
 (segment (start 85.5224 73.38) (end 85.5224 70.9924) (width 0.4) (layer "B.Cu") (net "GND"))
 (segment (start 94.8436 71.0184) (end 94.8944 70.9676) (width 0.4) (layer "B.Cu") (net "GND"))
 (segment (start 102.108 76.6064) (end 101.346 77.3684) (width 0.4) (layer "B.Cu") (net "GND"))
 (segment (start 76.3524 70.9676) (end 85.5472 70.9676) (width 0.4) (layer "B.Cu") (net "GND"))
 (segment (start 66.88 73.38) (end 66.88 71.4484) (width 0.4) (layer "B.Cu") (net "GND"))
 (segment (start 102.108 71.7804) (end 102.108 76.6064) (width 0.4) (layer "B.Cu") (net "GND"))
 (segment (start 76.2012 73.38) (end 76.2012 71.1188) (width 0.4) (layer "B.Cu") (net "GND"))
 (segment (start 85.5224 70.9924) (end 85.5472 70.9676) (width 0.4) (layer "B.Cu") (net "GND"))
 (segment (start 85.5472 70.9676) (end 94.8944 70.9676) (width 0.4) (layer "B.Cu") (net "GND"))
 (segment (start 67.3608 70.9676) (end 76.3524 70.9676) (width 0.4) (layer "B.Cu") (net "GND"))
 (segment (start 66.88 73.38) (end 66.88 77.3684) (width 0.4) (layer "B.Cu") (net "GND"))
 (segment (start 94.8436 73.38) (end 94.8436 71.0184) (width 0.4) (layer "B.Cu") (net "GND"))
 (segment (start 101.2952 70.9676) (end 102.108 71.7804) (width 0.4) (layer "B.Cu") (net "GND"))
 (segment (start 76.2012 71.1188) (end 76.3524 70.9676) (width 0.4) (layer "B.Cu") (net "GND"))
 (segment (start 94.8944 70.9676) (end 101.2952 70.9676) (width 0.4) (layer "B.Cu") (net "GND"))
 (segment (start 101.346 77.3684) (end 99.9744 77.3684) (width 0.4) (layer "B.Cu") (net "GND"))
 (segment (start 66.88 71.4484) (end 67.3608 70.9676) (width 0.4) (layer "B.Cu") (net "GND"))
 (segment (start 81.2812 73.38) (end 81.2812 74.8296) (width 0.4) (layer "B.Cu") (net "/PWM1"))
 (segment (start 91.8368 75.7332) (end 92.3544 76.2508) (width 0.4) (layer "B.Cu") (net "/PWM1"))
 (segment (start 81.2812 74.8296) (end 82.1848 75.7332) (width 0.4) (layer "B.Cu") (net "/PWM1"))
 (segment (start 92.3544 76.2508) (end 92.3544 77.3684) (width 0.4) (layer "B.Cu") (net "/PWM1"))
 (segment (start 82.1848 75.7332) (end 91.8368 75.7332) (width 0.4) (layer "B.Cu") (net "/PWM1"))
 (segment (start 94.4372 75.7936) (end 93.0656 75.7936) (width 0.4) (layer "B.Cu") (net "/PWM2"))
 (segment (start 94.8944 77.3684) (end 94.553872 77.3684) (width 0.4) (layer "B.Cu") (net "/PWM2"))
 (segment (start 90.6024 73.416928) (end 90.6024 73.38) (width 0.4) (layer "B.Cu") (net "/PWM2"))
 (segment (start 94.8944 77.3684) (end 94.8944 76.2508) (width 0.4) (layer "B.Cu") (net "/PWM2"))
 (segment (start 90.652 73.38) (end 90.6024 73.38) (width 0.4) (layer "B.Cu") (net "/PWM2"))
 (segment (start 93.0656 75.7936) (end 90.652 73.38) (width 0.4) (layer "B.Cu") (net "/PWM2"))
 (segment (start 94.8944 76.2508) (end 94.4372 75.7936) (width 0.4) (layer "B.Cu") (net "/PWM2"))
 (segment (start 97.9932 75.2348) (end 97.4344 75.7936) (width 0.4) (layer "B.Cu") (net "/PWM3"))
 (segment (start 97.4344 75.7936) (end 97.4344 77.3684) (width 0.4) (layer "B.Cu") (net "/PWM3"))
 (segment (start 99.5172 75.2348) (end 97.9932 75.2348) (width 0.4) (layer "B.Cu") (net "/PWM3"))
 (segment (start 99.9236 74.8284) (end 99.5172 75.2348) (width 0.4) (layer "B.Cu") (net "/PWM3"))
 (segment (start 99.9236 73.38) (end 99.9236 74.8284) (width 0.4) (layer "B.Cu") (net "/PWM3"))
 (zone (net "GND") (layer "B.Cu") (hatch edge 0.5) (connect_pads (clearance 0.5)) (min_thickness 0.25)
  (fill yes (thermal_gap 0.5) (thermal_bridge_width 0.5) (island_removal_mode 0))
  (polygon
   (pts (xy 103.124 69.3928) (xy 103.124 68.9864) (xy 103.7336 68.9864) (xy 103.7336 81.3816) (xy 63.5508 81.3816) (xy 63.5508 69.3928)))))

